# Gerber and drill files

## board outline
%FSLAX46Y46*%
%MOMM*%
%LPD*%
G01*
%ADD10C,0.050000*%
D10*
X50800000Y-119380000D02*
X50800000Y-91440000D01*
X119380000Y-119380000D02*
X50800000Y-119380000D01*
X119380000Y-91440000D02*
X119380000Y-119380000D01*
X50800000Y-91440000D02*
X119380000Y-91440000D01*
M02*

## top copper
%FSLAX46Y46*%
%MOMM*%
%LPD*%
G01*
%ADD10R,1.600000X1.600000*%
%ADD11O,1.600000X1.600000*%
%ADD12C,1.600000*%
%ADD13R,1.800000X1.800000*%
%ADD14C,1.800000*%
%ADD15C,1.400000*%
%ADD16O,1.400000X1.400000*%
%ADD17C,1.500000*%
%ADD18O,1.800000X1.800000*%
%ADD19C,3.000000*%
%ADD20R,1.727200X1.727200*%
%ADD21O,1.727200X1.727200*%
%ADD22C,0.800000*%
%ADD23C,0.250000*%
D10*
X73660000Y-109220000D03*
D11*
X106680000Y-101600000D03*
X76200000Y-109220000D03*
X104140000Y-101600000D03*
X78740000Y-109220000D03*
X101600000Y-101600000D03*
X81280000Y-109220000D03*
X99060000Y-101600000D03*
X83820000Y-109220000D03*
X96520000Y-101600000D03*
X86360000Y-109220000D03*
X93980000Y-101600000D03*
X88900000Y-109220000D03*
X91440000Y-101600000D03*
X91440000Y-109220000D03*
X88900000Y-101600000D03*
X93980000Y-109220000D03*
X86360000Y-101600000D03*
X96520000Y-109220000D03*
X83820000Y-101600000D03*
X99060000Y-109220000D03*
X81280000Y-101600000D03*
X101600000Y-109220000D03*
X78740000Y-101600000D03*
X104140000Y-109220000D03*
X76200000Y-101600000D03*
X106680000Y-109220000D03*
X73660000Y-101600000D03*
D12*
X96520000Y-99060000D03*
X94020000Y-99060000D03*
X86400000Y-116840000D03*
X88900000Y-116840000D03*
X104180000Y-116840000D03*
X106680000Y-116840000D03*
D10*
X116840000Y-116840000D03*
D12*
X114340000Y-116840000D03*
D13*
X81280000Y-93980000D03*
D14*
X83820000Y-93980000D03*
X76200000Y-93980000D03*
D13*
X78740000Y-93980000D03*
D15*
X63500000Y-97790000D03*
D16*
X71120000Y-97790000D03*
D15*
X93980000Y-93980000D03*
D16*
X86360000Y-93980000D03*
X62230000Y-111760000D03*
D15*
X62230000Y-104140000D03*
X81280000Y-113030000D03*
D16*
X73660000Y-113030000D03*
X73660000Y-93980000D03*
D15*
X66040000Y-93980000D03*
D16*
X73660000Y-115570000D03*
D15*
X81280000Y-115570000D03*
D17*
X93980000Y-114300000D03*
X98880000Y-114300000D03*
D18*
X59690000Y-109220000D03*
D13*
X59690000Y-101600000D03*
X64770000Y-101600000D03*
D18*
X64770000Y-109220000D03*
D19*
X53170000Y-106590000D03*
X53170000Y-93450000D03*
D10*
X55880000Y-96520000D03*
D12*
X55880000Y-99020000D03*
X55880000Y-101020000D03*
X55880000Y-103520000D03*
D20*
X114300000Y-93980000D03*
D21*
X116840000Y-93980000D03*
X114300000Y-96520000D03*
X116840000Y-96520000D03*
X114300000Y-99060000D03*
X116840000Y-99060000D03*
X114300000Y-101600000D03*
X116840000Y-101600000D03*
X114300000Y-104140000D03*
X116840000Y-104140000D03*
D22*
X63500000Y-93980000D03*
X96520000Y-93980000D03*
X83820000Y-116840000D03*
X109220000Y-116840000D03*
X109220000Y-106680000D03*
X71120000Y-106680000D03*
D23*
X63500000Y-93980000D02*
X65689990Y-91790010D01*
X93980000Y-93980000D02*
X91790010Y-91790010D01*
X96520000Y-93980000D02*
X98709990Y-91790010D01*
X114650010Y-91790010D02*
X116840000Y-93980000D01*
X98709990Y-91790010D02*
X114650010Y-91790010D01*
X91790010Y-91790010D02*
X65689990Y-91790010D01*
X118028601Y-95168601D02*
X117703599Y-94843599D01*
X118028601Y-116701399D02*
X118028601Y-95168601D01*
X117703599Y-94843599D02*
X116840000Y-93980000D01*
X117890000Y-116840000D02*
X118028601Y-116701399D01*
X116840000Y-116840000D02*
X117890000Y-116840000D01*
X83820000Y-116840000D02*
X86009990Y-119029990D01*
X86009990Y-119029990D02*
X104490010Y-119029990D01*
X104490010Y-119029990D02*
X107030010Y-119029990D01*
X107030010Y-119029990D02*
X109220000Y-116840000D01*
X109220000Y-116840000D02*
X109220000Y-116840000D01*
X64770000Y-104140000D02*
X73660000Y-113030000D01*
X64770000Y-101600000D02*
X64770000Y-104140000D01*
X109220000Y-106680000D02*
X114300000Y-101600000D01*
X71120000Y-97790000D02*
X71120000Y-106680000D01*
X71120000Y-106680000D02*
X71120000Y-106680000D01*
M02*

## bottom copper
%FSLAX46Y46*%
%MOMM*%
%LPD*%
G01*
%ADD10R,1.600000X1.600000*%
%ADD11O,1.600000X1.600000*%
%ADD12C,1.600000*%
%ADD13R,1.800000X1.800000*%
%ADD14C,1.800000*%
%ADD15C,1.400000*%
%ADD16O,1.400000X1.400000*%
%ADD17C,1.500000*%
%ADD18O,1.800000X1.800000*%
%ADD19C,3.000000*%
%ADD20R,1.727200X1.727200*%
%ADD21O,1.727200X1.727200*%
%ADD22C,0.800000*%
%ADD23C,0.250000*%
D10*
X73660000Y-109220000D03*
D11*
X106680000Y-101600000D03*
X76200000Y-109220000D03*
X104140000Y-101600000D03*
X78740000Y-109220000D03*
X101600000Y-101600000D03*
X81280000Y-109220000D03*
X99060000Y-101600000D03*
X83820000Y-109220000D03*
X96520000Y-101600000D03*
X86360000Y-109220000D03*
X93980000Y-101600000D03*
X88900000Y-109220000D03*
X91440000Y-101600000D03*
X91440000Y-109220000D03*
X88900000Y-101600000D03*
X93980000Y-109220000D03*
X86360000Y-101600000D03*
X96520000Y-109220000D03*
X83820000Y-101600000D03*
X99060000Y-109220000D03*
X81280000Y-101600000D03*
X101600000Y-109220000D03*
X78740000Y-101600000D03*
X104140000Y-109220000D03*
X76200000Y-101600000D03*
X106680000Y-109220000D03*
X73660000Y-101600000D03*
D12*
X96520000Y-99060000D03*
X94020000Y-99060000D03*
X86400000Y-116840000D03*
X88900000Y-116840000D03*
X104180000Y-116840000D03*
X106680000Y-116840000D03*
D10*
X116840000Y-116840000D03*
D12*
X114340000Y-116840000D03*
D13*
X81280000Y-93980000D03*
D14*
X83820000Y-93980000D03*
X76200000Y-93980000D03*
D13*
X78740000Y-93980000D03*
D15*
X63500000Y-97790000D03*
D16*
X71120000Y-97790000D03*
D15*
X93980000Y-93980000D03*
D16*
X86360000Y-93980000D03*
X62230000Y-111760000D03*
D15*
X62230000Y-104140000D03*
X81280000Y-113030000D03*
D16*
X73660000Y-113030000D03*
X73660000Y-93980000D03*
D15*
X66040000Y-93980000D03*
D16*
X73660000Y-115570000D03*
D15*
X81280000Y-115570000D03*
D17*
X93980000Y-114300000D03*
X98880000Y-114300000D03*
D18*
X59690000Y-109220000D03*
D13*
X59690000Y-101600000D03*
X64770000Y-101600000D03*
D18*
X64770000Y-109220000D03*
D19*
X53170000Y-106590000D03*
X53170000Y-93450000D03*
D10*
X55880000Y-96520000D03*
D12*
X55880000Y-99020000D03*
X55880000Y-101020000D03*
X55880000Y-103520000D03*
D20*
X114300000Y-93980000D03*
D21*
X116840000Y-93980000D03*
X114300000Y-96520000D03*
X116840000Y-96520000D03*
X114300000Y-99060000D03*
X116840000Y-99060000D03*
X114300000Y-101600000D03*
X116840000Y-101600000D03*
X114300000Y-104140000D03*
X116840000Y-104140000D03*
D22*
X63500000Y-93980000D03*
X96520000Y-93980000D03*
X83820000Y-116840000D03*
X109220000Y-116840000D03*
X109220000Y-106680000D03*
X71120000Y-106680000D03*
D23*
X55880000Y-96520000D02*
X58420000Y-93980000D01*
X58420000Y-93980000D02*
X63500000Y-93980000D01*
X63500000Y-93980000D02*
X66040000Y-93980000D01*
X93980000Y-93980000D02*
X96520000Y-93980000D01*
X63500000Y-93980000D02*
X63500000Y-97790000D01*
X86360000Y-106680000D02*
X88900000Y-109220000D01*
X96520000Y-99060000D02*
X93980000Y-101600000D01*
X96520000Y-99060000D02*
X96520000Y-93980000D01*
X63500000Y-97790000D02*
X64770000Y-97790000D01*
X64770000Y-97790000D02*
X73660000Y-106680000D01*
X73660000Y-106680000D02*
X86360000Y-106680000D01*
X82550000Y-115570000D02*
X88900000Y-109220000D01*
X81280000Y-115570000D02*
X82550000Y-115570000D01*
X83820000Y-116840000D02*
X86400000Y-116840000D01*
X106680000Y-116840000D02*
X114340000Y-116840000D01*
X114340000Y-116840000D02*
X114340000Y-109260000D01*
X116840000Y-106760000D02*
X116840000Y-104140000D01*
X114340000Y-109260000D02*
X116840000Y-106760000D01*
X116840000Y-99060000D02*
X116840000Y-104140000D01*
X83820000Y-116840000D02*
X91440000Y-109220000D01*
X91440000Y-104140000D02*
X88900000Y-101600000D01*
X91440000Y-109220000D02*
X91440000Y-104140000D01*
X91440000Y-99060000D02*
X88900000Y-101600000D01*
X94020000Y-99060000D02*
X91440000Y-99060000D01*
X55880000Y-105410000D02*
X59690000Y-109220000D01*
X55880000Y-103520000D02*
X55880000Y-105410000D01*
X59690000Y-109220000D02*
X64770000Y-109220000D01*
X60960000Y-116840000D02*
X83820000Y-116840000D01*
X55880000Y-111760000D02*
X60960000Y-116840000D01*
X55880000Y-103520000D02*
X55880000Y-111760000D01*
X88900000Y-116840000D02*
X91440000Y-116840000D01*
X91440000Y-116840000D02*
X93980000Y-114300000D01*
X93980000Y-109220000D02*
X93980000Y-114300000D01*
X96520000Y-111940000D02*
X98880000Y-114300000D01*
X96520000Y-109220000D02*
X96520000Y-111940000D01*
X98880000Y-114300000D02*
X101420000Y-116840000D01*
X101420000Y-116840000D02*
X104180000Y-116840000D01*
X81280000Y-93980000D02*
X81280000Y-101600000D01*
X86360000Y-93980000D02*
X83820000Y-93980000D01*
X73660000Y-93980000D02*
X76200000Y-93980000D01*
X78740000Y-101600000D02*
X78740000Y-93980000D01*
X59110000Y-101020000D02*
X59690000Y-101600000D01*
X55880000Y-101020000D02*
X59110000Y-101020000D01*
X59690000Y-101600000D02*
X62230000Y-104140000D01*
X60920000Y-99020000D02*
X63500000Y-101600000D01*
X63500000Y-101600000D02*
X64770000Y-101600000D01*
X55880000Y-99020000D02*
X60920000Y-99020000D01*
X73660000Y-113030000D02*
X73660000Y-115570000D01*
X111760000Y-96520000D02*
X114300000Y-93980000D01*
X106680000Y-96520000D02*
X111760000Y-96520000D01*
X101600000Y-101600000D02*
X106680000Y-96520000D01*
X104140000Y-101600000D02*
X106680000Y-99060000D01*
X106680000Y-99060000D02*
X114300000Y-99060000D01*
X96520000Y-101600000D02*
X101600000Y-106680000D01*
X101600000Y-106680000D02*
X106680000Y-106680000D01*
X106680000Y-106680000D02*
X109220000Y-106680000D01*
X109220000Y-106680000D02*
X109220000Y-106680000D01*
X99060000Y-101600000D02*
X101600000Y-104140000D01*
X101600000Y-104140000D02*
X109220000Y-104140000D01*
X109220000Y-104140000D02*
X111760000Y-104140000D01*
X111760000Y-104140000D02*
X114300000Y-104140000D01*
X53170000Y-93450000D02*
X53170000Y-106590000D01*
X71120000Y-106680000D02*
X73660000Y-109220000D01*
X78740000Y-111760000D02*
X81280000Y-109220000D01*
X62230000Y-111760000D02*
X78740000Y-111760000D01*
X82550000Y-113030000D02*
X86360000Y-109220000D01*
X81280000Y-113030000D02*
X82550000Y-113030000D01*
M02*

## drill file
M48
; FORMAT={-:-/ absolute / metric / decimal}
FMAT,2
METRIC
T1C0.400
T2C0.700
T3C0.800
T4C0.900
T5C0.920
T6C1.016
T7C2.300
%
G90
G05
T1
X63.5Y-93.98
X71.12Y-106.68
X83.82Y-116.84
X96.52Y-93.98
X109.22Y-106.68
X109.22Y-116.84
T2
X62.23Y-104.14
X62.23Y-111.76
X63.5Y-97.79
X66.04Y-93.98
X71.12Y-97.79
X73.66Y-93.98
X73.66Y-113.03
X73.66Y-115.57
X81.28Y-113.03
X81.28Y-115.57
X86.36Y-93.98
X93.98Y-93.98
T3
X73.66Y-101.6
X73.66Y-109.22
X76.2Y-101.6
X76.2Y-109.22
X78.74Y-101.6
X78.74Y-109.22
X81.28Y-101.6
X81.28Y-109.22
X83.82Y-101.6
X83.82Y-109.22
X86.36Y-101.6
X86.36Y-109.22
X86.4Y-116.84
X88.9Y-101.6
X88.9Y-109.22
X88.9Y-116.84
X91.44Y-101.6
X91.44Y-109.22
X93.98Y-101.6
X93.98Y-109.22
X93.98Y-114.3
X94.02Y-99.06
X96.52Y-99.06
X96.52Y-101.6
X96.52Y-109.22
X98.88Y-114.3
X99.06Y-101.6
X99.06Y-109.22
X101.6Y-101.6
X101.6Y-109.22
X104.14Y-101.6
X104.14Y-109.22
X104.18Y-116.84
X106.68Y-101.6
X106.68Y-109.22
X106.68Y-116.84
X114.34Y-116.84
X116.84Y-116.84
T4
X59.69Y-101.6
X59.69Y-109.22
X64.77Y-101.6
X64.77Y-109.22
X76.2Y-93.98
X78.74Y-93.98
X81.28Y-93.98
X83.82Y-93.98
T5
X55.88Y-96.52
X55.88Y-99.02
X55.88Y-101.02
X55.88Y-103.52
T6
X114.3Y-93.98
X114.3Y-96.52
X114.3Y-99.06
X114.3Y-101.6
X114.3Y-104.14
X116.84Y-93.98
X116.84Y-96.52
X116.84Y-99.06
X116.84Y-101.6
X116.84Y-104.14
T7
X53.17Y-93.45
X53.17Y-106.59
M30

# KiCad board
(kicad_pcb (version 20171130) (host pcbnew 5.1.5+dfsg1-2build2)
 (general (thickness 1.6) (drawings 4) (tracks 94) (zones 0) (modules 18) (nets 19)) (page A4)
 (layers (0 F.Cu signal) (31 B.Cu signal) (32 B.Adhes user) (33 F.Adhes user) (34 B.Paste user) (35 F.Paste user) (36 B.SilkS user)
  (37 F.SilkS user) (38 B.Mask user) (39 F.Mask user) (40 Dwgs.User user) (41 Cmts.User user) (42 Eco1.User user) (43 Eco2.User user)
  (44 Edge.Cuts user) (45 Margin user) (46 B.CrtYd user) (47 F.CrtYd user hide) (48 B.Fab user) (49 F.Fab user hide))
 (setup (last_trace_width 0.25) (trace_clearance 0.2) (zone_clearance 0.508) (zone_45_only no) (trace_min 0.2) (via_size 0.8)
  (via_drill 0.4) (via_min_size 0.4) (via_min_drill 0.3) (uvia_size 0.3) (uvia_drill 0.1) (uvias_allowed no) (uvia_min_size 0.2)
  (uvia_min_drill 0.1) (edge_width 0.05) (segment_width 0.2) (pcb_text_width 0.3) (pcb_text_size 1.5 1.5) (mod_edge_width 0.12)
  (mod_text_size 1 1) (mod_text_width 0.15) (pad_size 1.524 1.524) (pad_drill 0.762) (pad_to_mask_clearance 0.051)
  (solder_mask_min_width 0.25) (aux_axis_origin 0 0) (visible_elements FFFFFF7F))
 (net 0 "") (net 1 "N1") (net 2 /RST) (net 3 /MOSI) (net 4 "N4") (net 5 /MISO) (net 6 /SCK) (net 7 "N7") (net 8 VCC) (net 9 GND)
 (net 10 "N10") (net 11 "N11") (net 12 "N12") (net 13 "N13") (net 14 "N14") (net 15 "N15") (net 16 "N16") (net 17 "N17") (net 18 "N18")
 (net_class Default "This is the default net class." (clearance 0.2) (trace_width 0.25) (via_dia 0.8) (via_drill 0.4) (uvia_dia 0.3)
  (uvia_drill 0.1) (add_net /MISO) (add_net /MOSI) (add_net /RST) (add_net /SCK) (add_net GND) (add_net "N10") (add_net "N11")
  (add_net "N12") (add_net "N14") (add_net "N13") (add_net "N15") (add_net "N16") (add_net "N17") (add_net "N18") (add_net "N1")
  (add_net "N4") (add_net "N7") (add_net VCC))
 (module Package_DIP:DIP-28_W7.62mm (layer F.Cu) (at 73.66 109.22 90)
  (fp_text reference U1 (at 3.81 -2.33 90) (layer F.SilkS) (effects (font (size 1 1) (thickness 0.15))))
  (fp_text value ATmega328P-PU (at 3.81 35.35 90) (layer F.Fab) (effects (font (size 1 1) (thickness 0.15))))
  (pad 1 thru_hole rect (at 0 0 90) (size 1.6 1.6) (drill 0.8) (layers *.Cu *.Mask) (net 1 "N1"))
  (pad 15 thru_hole oval (at 7.62 33.02 90) (size 1.6 1.6) (drill 0.8) (layers *.Cu *.Mask))
  (pad 2 thru_hole oval (at 0 2.54 90) (size 1.6 1.6) (drill 0.8) (layers *.Cu *.Mask))
  (pad 16 thru_hole oval (at 7.62 30.48 90) (size 1.6 1.6) (drill 0.8) (layers *.Cu *.Mask) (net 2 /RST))
  (pad 3 thru_hole oval (at 0 5.08 90) (size 1.6 1.6) (drill 0.8) (layers *.Cu *.Mask))
  (pad 17 thru_hole oval (at 7.62 27.94 90) (size 1.6 1.6) (drill 0.8) (layers *.Cu *.Mask) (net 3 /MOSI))
  (pad 4 thru_hole oval (at 0 7.62 90) (size 1.6 1.6) (drill 0.8) (layers *.Cu *.Mask) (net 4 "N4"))
  (pad 18 thru_hole oval (at 7.62 25.4 90) (size 1.6 1.6) (drill 0.8) (layers *.Cu *.Mask) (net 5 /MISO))
  (pad 5 thru_hole oval (at 0 10.16 90) (size 1.6 1.6) (drill 0.8) (layers *.Cu *.Mask))
  (pad 19 thru_hole oval (at 7.62 22.86 90) (size 1.6 1.6) (drill 0.8) (layers *.Cu *.Mask) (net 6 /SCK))
  (pad 6 thru_hole oval (at 0 12.7 90) (size 1.6 1.6) (drill 0.8) (layers *.Cu *.Mask) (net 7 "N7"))
  (pad 20 thru_hole oval (at 7.62 20.32 90) (size 1.6 1.6) (drill 0.8) (layers *.Cu *.Mask) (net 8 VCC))
  (pad 7 thru_hole oval (at 0 15.24 90) (size 1.6 1.6) (drill 0.8) (layers *.Cu *.Mask) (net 8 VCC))
  (pad 21 thru_hole oval (at 7.62 17.78 90) (size 1.6 1.6) (drill 0.8) (layers *.Cu *.Mask))
  (pad 8 thru_hole oval (at 0 17.78 90) (size 1.6 1.6) (drill 0.8) (layers *.Cu *.Mask) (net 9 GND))
  (pad 22 thru_hole oval (at 7.62 15.24 90) (size 1.6 1.6) (drill 0.8) (layers *.Cu *.Mask) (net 9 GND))
  (pad 9 thru_hole oval (at 0 20.32 90) (size 1.6 1.6) (drill 0.8) (layers *.Cu *.Mask) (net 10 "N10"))
  (pad 23 thru_hole oval (at 7.62 12.7 90) (size 1.6 1.6) (drill 0.8) (layers *.Cu *.Mask))
  (pad 10 thru_hole oval (at 0 22.86 90) (size 1.6 1.6) (drill 0.8) (layers *.Cu *.Mask) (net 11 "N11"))
  (pad 24 thru_hole oval (at 7.62 10.16 90) (size 1.6 1.6) (drill 0.8) (layers *.Cu *.Mask))
  (pad 11 thru_hole oval (at 0 25.4 90) (size 1.6 1.6) (drill 0.8) (layers *.Cu *.Mask))
  (pad 25 thru_hole oval (at 7.62 7.62 90) (size 1.6 1.6) (drill 0.8) (layers *.Cu *.Mask) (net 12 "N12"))
  (pad 12 thru_hole oval (at 0 27.94 90) (size 1.6 1.6) (drill 0.8) (layers *.Cu *.Mask))
  (pad 26 thru_hole oval (at 7.62 5.08 90) (size 1.6 1.6) (drill 0.8) (layers *.Cu *.Mask) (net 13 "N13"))
  (pad 13 thru_hole oval (at 0 30.48 90) (size 1.6 1.6) (drill 0.8) (layers *.Cu *.Mask))
  (pad 27 thru_hole oval (at 7.62 2.54 90) (size 1.6 1.6) (drill 0.8) (layers *.Cu *.Mask))
  (pad 14 thru_hole oval (at 0 33.02 90) (size 1.6 1.6) (drill 0.8) (layers *.Cu *.Mask))
  (pad 28 thru_hole oval (at 7.62 0 90) (size 1.6 1.6) (drill 0.8) (layers *.Cu *.Mask)))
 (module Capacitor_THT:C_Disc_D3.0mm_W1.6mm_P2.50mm (layer F.Cu) (at 96.52 99.06 180)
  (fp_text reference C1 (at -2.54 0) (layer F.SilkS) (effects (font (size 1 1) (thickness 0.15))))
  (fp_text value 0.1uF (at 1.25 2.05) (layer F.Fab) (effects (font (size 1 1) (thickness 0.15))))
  (pad 1 thru_hole circle (at 0 0 180) (size 1.6 1.6) (drill 0.8) (layers *.Cu *.Mask) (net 8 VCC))
  (pad 2 thru_hole circle (at 2.5 0 180) (size 1.6 1.6) (drill 0.8) (layers *.Cu *.Mask) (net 9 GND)))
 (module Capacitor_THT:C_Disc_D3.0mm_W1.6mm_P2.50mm (layer F.Cu) (at 88.9 116.84 180)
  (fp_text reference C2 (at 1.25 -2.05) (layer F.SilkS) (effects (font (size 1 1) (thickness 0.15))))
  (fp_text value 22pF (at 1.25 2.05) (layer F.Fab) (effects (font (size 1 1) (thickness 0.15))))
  (pad 2 thru_hole circle (at 2.5 0 180) (size 1.6 1.6) (drill 0.8) (layers *.Cu *.Mask) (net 9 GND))
  (pad 1 thru_hole circle (at 0 0 180) (size 1.6 1.6) (drill 0.8) (layers *.Cu *.Mask) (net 10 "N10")))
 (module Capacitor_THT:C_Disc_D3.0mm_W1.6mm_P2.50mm (layer F.Cu) (at 104.18 116.84)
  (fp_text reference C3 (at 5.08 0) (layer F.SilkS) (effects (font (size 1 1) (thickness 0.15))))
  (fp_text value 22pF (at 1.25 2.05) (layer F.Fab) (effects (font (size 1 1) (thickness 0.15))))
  (pad 1 thru_hole circle (at 0 0) (size 1.6 1.6) (drill 0.8) (layers *.Cu *.Mask) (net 11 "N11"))
  (pad 2 thru_hole circle (at 2.5 0) (size 1.6 1.6) (drill 0.8) (layers *.Cu *.Mask) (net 9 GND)))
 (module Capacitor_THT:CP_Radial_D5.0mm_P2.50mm (layer F.Cu) (at 116.84 116.84 180)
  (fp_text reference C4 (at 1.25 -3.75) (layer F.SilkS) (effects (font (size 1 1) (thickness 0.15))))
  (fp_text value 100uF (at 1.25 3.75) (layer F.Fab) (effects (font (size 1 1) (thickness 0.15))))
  (pad 1 thru_hole rect (at 0 0 180) (size 1.6 1.6) (drill 0.8) (layers *.Cu *.Mask) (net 8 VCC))
  (pad 2 thru_hole circle (at 2.5 0 180) (size 1.6 1.6) (drill 0.8) (layers *.Cu *.Mask) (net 9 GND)))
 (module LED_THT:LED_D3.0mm (layer F.Cu) (at 81.28 93.98)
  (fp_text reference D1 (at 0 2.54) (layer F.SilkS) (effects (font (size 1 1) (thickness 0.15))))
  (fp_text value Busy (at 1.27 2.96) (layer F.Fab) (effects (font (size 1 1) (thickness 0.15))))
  (pad 1 thru_hole rect (at 0 0) (size 1.8 1.8) (drill 0.9) (layers *.Cu *.Mask) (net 12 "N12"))
  (pad 2 thru_hole circle (at 2.54 0) (size 1.8 1.8) (drill 0.9) (layers *.Cu *.Mask) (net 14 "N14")))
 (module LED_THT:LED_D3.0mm (layer F.Cu) (at 78.74 93.98 180)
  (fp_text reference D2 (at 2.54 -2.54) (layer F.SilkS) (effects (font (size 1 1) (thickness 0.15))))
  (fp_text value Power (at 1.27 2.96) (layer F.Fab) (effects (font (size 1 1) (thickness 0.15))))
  (pad 2 thru_hole circle (at 2.54 0 180) (size 1.8 1.8) (drill 0.9) (layers *.Cu *.Mask) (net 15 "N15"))
  (pad 1 thru_hole rect (at 0 0 180) (size 1.8 1.8) (drill 0.9) (layers *.Cu *.Mask) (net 13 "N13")))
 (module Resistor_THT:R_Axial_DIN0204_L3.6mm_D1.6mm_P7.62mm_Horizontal (layer F.Cu) (at 63.5 97.79)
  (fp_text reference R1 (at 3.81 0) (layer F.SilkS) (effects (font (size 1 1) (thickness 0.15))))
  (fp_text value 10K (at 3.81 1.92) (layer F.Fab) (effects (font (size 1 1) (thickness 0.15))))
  (pad 1 thru_hole circle (at 0 0) (size 1.4 1.4) (drill 0.7) (layers *.Cu *.Mask) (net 8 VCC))
  (pad 2 thru_hole oval (at 7.62 0) (size 1.4 1.4) (drill 0.7) (layers *.Cu *.Mask) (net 1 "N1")))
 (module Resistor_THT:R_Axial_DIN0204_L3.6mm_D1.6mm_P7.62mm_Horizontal (layer F.Cu) (at 93.98 93.98 180)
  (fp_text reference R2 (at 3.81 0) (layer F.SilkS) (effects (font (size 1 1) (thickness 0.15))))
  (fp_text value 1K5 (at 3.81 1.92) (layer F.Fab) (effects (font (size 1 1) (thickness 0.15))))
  (pad 1 thru_hole circle (at 0 0 180) (size 1.4 1.4) (drill 0.7) (layers *.Cu *.Mask) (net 8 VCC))
  (pad 2 thru_hole oval (at 7.62 0 180) (size 1.4 1.4) (drill 0.7) (layers *.Cu *.Mask) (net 14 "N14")))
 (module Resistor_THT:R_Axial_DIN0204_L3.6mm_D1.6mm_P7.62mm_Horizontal (layer F.Cu) (at 62.23 104.14 270)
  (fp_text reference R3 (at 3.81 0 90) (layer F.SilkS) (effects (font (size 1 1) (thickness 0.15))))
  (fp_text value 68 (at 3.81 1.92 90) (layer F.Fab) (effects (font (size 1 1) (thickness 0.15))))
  (pad 2 thru_hole oval (at 7.62 0 270) (size 1.4 1.4) (drill 0.7) (layers *.Cu *.Mask) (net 4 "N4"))
  (pad 1 thru_hole circle (at 0 0 270) (size 1.4 1.4) (drill 0.7) (layers *.Cu *.Mask) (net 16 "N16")))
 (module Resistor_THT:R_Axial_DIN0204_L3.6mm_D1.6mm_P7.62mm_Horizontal (layer F.Cu) (at 81.28 113.03 180)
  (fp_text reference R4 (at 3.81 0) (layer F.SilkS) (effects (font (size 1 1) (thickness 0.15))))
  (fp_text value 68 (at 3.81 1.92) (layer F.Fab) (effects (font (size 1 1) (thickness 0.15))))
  (pad 1 thru_hole circle (at 0 0 180) (size 1.4 1.4) (drill 0.7) (layers *.Cu *.Mask) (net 7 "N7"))
  (pad 2 thru_hole oval (at 7.62 0 180) (size 1.4 1.4) (drill 0.7) (layers *.Cu *.Mask) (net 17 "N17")))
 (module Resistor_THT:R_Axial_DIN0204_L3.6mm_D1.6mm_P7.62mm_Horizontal (layer F.Cu) (at 66.04 93.98)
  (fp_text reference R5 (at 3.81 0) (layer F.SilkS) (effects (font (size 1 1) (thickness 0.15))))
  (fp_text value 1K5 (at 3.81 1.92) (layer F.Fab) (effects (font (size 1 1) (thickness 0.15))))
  (pad 2 thru_hole oval (at 7.62 0) (size 1.4 1.4) (drill 0.7) (layers *.Cu *.Mask) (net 15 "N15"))
  (pad 1 thru_hole circle (at 0 0) (size 1.4 1.4) (drill 0.7) (layers *.Cu *.Mask) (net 8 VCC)))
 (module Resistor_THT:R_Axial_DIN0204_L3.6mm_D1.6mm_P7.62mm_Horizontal (layer F.Cu) (at 81.28 115.57 180)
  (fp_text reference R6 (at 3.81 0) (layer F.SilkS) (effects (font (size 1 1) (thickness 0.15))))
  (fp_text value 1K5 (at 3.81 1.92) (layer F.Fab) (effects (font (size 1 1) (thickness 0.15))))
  (pad 2 thru_hole oval (at 7.62 0 180) (size 1.4 1.4) (drill 0.7) (layers *.Cu *.Mask) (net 17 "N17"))
  (pad 1 thru_hole circle (at 0 0 180) (size 1.4 1.4) (drill 0.7) (layers *.Cu *.Mask) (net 8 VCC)))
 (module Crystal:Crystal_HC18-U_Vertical (layer F.Cu) (at 93.98 114.3)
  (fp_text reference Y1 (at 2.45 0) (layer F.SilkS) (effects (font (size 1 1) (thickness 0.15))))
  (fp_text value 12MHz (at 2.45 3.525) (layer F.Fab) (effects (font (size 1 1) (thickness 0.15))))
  (pad 1 thru_hole circle (at 0 0) (size 1.5 1.5) (drill 0.8) (layers *.Cu *.Mask) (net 10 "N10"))
  (pad 2 thru_hole circle (at 4.9 0) (size 1.5 1.5) (drill 0.8) (layers *.Cu *.Mask) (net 11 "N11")))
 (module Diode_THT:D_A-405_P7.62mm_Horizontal (layer F.Cu) (at 59.69 101.6 270)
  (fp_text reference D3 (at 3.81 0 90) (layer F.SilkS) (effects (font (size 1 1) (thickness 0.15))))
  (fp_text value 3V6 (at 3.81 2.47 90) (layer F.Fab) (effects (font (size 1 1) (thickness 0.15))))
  (pad 2 thru_hole oval (at 7.62 0 270) (size 1.8 1.8) (drill 0.9) (layers *.Cu *.Mask) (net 9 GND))
  (pad 1 thru_hole rect (at 0 0 270) (size 1.8 1.8) (drill 0.9) (layers *.Cu *.Mask) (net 16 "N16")))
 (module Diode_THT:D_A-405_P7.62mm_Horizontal (layer F.Cu) (at 64.77 101.6 270)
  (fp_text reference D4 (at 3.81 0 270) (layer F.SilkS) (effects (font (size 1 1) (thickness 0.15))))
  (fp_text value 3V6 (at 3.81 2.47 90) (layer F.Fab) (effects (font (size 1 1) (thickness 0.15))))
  (pad 1 thru_hole rect (at 0 0 270) (size 1.8 1.8) (drill 0.9) (layers *.Cu *.Mask) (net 17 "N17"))
  (pad 2 thru_hole oval (at 7.62 0 270) (size 1.8 1.8) (drill 0.9) (layers *.Cu *.Mask) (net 9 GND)))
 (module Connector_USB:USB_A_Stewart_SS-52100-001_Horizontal (layer F.Cu) (at 55.88 96.52 270)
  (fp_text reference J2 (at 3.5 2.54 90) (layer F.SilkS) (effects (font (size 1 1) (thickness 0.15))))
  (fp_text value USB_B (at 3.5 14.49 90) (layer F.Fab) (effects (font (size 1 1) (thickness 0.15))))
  (pad 5 thru_hole circle (at 10.07 2.71 270) (size 3 3) (drill 2.3) (layers *.Cu *.Mask) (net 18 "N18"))
  (pad 5 thru_hole circle (at -3.07 2.71 270) (size 3 3) (drill 2.3) (layers *.Cu *.Mask) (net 18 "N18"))
  (pad 1 thru_hole rect (at 0 0 270) (size 1.6 1.6) (drill 0.92) (layers *.Cu *.Mask) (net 8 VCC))
  (pad 2 thru_hole circle (at 2.5 0 270) (size 1.6 1.6) (drill 0.92) (layers *.Cu *.Mask) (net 17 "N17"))
  (pad 3 thru_hole circle (at 4.5 0 270) (size 1.6 1.6) (drill 0.92) (layers *.Cu *.Mask) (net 16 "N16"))
  (pad 4 thru_hole circle (at 7 0 270) (size 1.6 1.6) (drill 0.92) (layers *.Cu *.Mask) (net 9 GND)))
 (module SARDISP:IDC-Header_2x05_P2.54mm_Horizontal (layer F.Cu) (at 114.3 93.98)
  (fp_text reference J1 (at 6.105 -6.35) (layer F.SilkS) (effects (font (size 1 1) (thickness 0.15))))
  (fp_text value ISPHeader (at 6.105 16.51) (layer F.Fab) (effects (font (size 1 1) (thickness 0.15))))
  (pad 1 thru_hole rect (at 0 0) (size 1.7272 1.7272) (drill 1.016) (layers *.Cu *.Mask) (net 3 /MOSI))
  (pad 2 thru_hole oval (at 2.54 0) (size 1.7272 1.7272) (drill 1.016) (layers *.Cu *.Mask) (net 8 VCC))
  (pad 3 thru_hole oval (at 0 2.54) (size 1.7272 1.7272) (drill 1.016) (layers *.Cu *.Mask))
  (pad 4 thru_hole oval (at 2.54 2.54) (size 1.7272 1.7272) (drill 1.016) (layers *.Cu *.Mask))
  (pad 5 thru_hole oval (at 0 5.08) (size 1.7272 1.7272) (drill 1.016) (layers *.Cu *.Mask) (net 2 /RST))
  (pad 6 thru_hole oval (at 2.54 5.08) (size 1.7272 1.7272) (drill 1.016) (layers *.Cu *.Mask) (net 9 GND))
  (pad 7 thru_hole oval (at 0 7.62) (size 1.7272 1.7272) (drill 1.016) (layers *.Cu *.Mask) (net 6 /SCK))
  (pad 8 thru_hole oval (at 2.54 7.62) (size 1.7272 1.7272) (drill 1.016) (layers *.Cu *.Mask) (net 9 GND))
  (pad 9 thru_hole oval (at 0 10.16) (size 1.7272 1.7272) (drill 1.016) (layers *.Cu *.Mask) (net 5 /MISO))
  (pad 10 thru_hole oval (at 2.54 10.16) (size 1.7272 1.7272) (drill 1.016) (layers *.Cu *.Mask) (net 9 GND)))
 (gr_line (start 50.8 119.38) (end 50.8 91.44) (layer Edge.Cuts) (width 0.05))
 (gr_line (start 119.38 119.38) (end 50.8 119.38) (layer Edge.Cuts) (width 0.05))
 (gr_line (start 119.38 91.44) (end 119.38 119.38) (layer Edge.Cuts) (width 0.05))
 (gr_line (start 50.8 91.44) (end 119.38 91.44) (layer Edge.Cuts) (width 0.05))
 (segment (start 55.88 96.52) (end 58.42 93.98) (width 0.25) (layer B.Cu) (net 8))
 (segment (start 58.42 93.98) (end 63.5 93.98) (width 0.25) (layer B.Cu) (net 8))
 (segment (start 63.5 93.98) (end 66.04 93.98) (width 0.25) (layer B.Cu) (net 8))
 (via (at 63.5 93.98) (size 0.8) (drill 0.4) (layers F.Cu B.Cu) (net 8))
 (segment (start 63.5 93.98) (end 65.68999 91.79001) (width 0.25) (layer F.Cu) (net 8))
 (segment (start 93.98 93.98) (end 91.79001 91.79001) (width 0.25) (layer F.Cu) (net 8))
 (segment (start 93.98 93.98) (end 96.52 93.98) (width 0.25) (layer B.Cu) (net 8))
 (via (at 96.52 93.98) (size 0.8) (drill 0.4) (layers F.Cu B.Cu) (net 8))
 (segment (start 96.52 93.98) (end 98.70999 91.79001) (width 0.25) (layer F.Cu) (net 8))
 (segment (start 114.65001 91.79001) (end 116.84 93.98) (width 0.25) (layer F.Cu) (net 8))
 (segment (start 98.70999 91.79001) (end 114.65001 91.79001) (width 0.25) (layer F.Cu) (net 8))
 (segment (start 91.79001 91.79001) (end 65.68999 91.79001) (width 0.25) (layer F.Cu) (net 8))
 (segment (start 118.028601 95.168601) (end 117.703599 94.843599) (width 0.25) (layer F.Cu) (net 8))
 (segment (start 118.028601 116.701399) (end 118.028601 95.168601) (width 0.25) (layer F.Cu) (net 8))
 (segment (start 117.703599 94.843599) (end 116.84 93.98) (width 0.25) (layer F.Cu) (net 8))
 (segment (start 117.89 116.84) (end 118.028601 116.701399) (width 0.25) (layer F.Cu) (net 8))
 (segment (start 116.84 116.84) (end 117.89 116.84) (width 0.25) (layer F.Cu) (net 8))
 (segment (start 63.5 93.98) (end 63.5 97.79) (width 0.25) (layer B.Cu) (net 8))
 (segment (start 86.36 106.68) (end 88.9 109.22) (width 0.25) (layer B.Cu) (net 8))
 (segment (start 96.52 99.06) (end 93.98 101.6) (width 0.25) (layer B.Cu) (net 8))
 (segment (start 96.52 99.06) (end 96.52 93.98) (width 0.25) (layer B.Cu) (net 8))
 (segment (start 63.5 97.79) (end 64.77 97.79) (width 0.25) (layer B.Cu) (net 8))
 (segment (start 64.77 97.79) (end 73.66 106.68) (width 0.25) (layer B.Cu) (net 8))
 (segment (start 73.66 106.68) (end 86.36 106.68) (width 0.25) (layer B.Cu) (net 8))
 (segment (start 82.55 115.57) (end 88.9 109.22) (width 0.25) (layer B.Cu) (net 8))
 (segment (start 81.28 115.57) (end 82.55 115.57) (width 0.25) (layer B.Cu) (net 8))
 (segment (start 83.82 116.84) (end 86.4 116.84) (width 0.25) (layer B.Cu) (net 9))
 (via (at 83.82 116.84) (size 0.8) (drill 0.4) (layers F.Cu B.Cu) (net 9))
 (segment (start 83.82 116.84) (end 86.00999 119.02999) (width 0.25) (layer F.Cu) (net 9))
 (segment (start 106.68 116.84) (end 114.34 116.84) (width 0.25) (layer B.Cu) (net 9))
 (segment (start 86.00999 119.02999) (end 104.49001 119.02999) (width 0.25) (layer F.Cu) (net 9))
 (segment (start 104.49001 119.02999) (end 107.03001 119.02999) (width 0.25) (layer F.Cu) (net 9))
 (segment (start 107.03001 119.02999) (end 109.22 116.84) (width 0.25) (layer F.Cu) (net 9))
 (segment (start 109.22 116.84) (end 109.22 116.84) (width 0.25) (layer F.Cu) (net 9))
 (via (at 109.22 116.84) (size 0.8) (drill 0.4) (layers F.Cu B.Cu) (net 9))
 (segment (start 114.34 116.84) (end 114.34 109.26) (width 0.25) (layer B.Cu) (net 9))
 (segment (start 116.84 106.76) (end 116.84 104.14) (width 0.25) (layer B.Cu) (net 9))
 (segment (start 114.34 109.26) (end 116.84 106.76) (width 0.25) (layer B.Cu) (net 9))
 (segment (start 116.84 99.06) (end 116.84 104.14) (width 0.25) (layer B.Cu) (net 9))
 (segment (start 83.82 116.84) (end 91.44 109.22) (width 0.25) (layer B.Cu) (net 9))
 (segment (start 91.44 104.14) (end 88.9 101.6) (width 0.25) (layer B.Cu) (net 9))
 (segment (start 91.44 109.22) (end 91.44 104.14) (width 0.25) (layer B.Cu) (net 9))
 (segment (start 91.44 99.06) (end 88.9 101.6) (width 0.25) (layer B.Cu) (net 9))
 (segment (start 94.02 99.06) (end 91.44 99.06) (width 0.25) (layer B.Cu) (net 9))
 (segment (start 55.88 105.41) (end 59.69 109.22) (width 0.25) (layer B.Cu) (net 9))
 (segment (start 55.88 103.52) (end 55.88 105.41) (width 0.25) (layer B.Cu) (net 9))
 (segment (start 59.69 109.22) (end 64.77 109.22) (width 0.25) (layer B.Cu) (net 9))
 (segment (start 60.96 116.84) (end 83.82 116.84) (width 0.25) (layer B.Cu) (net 9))
 (segment (start 55.88 111.76) (end 60.96 116.84) (width 0.25) (layer B.Cu) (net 9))
 (segment (start 55.88 103.52) (end 55.88 111.76) (width 0.25) (layer B.Cu) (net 9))
 (segment (start 88.9 116.84) (end 91.44 116.84) (width 0.25) (layer B.Cu) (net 10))
 (segment (start 91.44 116.84) (end 93.98 114.3) (width 0.25) (layer B.Cu) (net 10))
 (segment (start 93.98 109.22) (end 93.98 114.3) (width 0.25) (layer B.Cu) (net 10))
 (segment (start 96.52 111.94) (end 98.88 114.3) (width 0.25) (layer B.Cu) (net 11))
 (segment (start 96.52 109.22) (end 96.52 111.94) (width 0.25) (layer B.Cu) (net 11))
 (segment (start 98.88 114.3) (end 101.42 116.84) (width 0.25) (layer B.Cu) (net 11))
 (segment (start 101.42 116.84) (end 104.18 116.84) (width 0.25) (layer B.Cu) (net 11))
 (segment (start 81.28 93.98) (end 81.28 101.6) (width 0.25) (layer B.Cu) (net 12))
 (segment (start 86.36 93.98) (end 83.82 93.98) (width 0.25) (layer B.Cu) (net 14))
 (segment (start 73.66 93.98) (end 76.2 93.98) (width 0.25) (layer B.Cu) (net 15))
 (segment (start 78.74 101.6) (end 78.74 93.98) (width 0.25) (layer B.Cu) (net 13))
 (segment (start 59.11 101.02) (end 59.69 101.6) (width 0.25) (layer B.Cu) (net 16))
 (segment (start 55.88 101.02) (end 59.11 101.02) (width 0.25) (layer B.Cu) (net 16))
 (segment (start 59.69 101.6) (end 62.23 104.14) (width 0.25) (layer B.Cu) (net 16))
 (segment (start 60.92 99.02) (end 63.5 101.6) (width 0.25) (layer B.Cu) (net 17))
 (segment (start 63.5 101.6) (end 64.77 101.6) (width 0.25) (layer B.Cu) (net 17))
 (segment (start 55.88 99.02) (end 60.92 99.02) (width 0.25) (layer B.Cu) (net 17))
 (segment (start 64.77 104.14) (end 73.66 113.03) (width 0.25) (layer F.Cu) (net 17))
 (segment (start 64.77 101.6) (end 64.77 104.14) (width 0.25) (layer F.Cu) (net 17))
 (segment (start 73.66 113.03) (end 73.66 115.57) (width 0.25) (layer B.Cu) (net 17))
 (segment (start 111.76 96.52) (end 114.3 93.98) (width 0.25) (layer B.Cu) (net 3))
 (segment (start 106.68 96.52) (end 111.76 96.52) (width 0.25) (layer B.Cu) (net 3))
 (segment (start 101.6 101.6) (end 106.68 96.52) (width 0.25) (layer B.Cu) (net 3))
 (segment (start 104.14 101.6) (end 106.68 99.06) (width 0.25) (layer B.Cu) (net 2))
 (segment (start 106.68 99.06) (end 114.3 99.06) (width 0.25) (layer B.Cu) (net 2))
 (segment (start 96.52 101.6) (end 101.6 106.68) (width 0.25) (layer B.Cu) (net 6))
 (segment (start 101.6 106.68) (end 106.68 106.68) (width 0.25) (layer B.Cu) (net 6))
 (segment (start 106.68 106.68) (end 109.22 106.68) (width 0.25) (layer B.Cu) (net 6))
 (segment (start 109.22 106.68) (end 109.22 106.68) (width 0.25) (layer B.Cu) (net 6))
 (via (at 109.22 106.68) (size 0.8) (drill 0.4) (layers F.Cu B.Cu) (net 6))
 (segment (start 109.22 106.68) (end 114.3 101.6) (width 0.25) (layer F.Cu) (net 6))
 (segment (start 99.06 101.6) (end 101.6 104.14) (width 0.25) (layer B.Cu) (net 5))
 (segment (start 101.6 104.14) (end 109.22 104.14) (width 0.25) (layer B.Cu) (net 5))
 (segment (start 109.22 104.14) (end 111.76 104.14) (width 0.25) (layer B.Cu) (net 5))
 (segment (start 111.76 104.14) (end 114.3 104.14) (width 0.25) (layer B.Cu) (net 5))
 (segment (start 53.17 93.45) (end 53.17 106.59) (width 0.25) (layer B.Cu) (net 18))
 (segment (start 71.12 97.79) (end 71.12 106.68) (width 0.25) (layer F.Cu) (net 1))
 (segment (start 71.12 106.68) (end 71.12 106.68) (width 0.25) (layer F.Cu) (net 1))
 (via (at 71.12 106.68) (size 0.8) (drill 0.4) (layers F.Cu B.Cu) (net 1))
 (segment (start 71.12 106.68) (end 73.66 109.22) (width 0.25) (layer B.Cu) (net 1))
 (segment (start 78.74 111.76) (end 81.28 109.22) (width 0.25) (layer B.Cu) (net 4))
 (segment (start 62.23 111.76) (end 78.74 111.76) (width 0.25) (layer B.Cu) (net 4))
 (segment (start 82.55 113.03) (end 86.36 109.22) (width 0.25) (layer B.Cu) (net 7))
 (segment (start 81.28 113.03) (end 82.55 113.03) (width 0.25) (layer B.Cu) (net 7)))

